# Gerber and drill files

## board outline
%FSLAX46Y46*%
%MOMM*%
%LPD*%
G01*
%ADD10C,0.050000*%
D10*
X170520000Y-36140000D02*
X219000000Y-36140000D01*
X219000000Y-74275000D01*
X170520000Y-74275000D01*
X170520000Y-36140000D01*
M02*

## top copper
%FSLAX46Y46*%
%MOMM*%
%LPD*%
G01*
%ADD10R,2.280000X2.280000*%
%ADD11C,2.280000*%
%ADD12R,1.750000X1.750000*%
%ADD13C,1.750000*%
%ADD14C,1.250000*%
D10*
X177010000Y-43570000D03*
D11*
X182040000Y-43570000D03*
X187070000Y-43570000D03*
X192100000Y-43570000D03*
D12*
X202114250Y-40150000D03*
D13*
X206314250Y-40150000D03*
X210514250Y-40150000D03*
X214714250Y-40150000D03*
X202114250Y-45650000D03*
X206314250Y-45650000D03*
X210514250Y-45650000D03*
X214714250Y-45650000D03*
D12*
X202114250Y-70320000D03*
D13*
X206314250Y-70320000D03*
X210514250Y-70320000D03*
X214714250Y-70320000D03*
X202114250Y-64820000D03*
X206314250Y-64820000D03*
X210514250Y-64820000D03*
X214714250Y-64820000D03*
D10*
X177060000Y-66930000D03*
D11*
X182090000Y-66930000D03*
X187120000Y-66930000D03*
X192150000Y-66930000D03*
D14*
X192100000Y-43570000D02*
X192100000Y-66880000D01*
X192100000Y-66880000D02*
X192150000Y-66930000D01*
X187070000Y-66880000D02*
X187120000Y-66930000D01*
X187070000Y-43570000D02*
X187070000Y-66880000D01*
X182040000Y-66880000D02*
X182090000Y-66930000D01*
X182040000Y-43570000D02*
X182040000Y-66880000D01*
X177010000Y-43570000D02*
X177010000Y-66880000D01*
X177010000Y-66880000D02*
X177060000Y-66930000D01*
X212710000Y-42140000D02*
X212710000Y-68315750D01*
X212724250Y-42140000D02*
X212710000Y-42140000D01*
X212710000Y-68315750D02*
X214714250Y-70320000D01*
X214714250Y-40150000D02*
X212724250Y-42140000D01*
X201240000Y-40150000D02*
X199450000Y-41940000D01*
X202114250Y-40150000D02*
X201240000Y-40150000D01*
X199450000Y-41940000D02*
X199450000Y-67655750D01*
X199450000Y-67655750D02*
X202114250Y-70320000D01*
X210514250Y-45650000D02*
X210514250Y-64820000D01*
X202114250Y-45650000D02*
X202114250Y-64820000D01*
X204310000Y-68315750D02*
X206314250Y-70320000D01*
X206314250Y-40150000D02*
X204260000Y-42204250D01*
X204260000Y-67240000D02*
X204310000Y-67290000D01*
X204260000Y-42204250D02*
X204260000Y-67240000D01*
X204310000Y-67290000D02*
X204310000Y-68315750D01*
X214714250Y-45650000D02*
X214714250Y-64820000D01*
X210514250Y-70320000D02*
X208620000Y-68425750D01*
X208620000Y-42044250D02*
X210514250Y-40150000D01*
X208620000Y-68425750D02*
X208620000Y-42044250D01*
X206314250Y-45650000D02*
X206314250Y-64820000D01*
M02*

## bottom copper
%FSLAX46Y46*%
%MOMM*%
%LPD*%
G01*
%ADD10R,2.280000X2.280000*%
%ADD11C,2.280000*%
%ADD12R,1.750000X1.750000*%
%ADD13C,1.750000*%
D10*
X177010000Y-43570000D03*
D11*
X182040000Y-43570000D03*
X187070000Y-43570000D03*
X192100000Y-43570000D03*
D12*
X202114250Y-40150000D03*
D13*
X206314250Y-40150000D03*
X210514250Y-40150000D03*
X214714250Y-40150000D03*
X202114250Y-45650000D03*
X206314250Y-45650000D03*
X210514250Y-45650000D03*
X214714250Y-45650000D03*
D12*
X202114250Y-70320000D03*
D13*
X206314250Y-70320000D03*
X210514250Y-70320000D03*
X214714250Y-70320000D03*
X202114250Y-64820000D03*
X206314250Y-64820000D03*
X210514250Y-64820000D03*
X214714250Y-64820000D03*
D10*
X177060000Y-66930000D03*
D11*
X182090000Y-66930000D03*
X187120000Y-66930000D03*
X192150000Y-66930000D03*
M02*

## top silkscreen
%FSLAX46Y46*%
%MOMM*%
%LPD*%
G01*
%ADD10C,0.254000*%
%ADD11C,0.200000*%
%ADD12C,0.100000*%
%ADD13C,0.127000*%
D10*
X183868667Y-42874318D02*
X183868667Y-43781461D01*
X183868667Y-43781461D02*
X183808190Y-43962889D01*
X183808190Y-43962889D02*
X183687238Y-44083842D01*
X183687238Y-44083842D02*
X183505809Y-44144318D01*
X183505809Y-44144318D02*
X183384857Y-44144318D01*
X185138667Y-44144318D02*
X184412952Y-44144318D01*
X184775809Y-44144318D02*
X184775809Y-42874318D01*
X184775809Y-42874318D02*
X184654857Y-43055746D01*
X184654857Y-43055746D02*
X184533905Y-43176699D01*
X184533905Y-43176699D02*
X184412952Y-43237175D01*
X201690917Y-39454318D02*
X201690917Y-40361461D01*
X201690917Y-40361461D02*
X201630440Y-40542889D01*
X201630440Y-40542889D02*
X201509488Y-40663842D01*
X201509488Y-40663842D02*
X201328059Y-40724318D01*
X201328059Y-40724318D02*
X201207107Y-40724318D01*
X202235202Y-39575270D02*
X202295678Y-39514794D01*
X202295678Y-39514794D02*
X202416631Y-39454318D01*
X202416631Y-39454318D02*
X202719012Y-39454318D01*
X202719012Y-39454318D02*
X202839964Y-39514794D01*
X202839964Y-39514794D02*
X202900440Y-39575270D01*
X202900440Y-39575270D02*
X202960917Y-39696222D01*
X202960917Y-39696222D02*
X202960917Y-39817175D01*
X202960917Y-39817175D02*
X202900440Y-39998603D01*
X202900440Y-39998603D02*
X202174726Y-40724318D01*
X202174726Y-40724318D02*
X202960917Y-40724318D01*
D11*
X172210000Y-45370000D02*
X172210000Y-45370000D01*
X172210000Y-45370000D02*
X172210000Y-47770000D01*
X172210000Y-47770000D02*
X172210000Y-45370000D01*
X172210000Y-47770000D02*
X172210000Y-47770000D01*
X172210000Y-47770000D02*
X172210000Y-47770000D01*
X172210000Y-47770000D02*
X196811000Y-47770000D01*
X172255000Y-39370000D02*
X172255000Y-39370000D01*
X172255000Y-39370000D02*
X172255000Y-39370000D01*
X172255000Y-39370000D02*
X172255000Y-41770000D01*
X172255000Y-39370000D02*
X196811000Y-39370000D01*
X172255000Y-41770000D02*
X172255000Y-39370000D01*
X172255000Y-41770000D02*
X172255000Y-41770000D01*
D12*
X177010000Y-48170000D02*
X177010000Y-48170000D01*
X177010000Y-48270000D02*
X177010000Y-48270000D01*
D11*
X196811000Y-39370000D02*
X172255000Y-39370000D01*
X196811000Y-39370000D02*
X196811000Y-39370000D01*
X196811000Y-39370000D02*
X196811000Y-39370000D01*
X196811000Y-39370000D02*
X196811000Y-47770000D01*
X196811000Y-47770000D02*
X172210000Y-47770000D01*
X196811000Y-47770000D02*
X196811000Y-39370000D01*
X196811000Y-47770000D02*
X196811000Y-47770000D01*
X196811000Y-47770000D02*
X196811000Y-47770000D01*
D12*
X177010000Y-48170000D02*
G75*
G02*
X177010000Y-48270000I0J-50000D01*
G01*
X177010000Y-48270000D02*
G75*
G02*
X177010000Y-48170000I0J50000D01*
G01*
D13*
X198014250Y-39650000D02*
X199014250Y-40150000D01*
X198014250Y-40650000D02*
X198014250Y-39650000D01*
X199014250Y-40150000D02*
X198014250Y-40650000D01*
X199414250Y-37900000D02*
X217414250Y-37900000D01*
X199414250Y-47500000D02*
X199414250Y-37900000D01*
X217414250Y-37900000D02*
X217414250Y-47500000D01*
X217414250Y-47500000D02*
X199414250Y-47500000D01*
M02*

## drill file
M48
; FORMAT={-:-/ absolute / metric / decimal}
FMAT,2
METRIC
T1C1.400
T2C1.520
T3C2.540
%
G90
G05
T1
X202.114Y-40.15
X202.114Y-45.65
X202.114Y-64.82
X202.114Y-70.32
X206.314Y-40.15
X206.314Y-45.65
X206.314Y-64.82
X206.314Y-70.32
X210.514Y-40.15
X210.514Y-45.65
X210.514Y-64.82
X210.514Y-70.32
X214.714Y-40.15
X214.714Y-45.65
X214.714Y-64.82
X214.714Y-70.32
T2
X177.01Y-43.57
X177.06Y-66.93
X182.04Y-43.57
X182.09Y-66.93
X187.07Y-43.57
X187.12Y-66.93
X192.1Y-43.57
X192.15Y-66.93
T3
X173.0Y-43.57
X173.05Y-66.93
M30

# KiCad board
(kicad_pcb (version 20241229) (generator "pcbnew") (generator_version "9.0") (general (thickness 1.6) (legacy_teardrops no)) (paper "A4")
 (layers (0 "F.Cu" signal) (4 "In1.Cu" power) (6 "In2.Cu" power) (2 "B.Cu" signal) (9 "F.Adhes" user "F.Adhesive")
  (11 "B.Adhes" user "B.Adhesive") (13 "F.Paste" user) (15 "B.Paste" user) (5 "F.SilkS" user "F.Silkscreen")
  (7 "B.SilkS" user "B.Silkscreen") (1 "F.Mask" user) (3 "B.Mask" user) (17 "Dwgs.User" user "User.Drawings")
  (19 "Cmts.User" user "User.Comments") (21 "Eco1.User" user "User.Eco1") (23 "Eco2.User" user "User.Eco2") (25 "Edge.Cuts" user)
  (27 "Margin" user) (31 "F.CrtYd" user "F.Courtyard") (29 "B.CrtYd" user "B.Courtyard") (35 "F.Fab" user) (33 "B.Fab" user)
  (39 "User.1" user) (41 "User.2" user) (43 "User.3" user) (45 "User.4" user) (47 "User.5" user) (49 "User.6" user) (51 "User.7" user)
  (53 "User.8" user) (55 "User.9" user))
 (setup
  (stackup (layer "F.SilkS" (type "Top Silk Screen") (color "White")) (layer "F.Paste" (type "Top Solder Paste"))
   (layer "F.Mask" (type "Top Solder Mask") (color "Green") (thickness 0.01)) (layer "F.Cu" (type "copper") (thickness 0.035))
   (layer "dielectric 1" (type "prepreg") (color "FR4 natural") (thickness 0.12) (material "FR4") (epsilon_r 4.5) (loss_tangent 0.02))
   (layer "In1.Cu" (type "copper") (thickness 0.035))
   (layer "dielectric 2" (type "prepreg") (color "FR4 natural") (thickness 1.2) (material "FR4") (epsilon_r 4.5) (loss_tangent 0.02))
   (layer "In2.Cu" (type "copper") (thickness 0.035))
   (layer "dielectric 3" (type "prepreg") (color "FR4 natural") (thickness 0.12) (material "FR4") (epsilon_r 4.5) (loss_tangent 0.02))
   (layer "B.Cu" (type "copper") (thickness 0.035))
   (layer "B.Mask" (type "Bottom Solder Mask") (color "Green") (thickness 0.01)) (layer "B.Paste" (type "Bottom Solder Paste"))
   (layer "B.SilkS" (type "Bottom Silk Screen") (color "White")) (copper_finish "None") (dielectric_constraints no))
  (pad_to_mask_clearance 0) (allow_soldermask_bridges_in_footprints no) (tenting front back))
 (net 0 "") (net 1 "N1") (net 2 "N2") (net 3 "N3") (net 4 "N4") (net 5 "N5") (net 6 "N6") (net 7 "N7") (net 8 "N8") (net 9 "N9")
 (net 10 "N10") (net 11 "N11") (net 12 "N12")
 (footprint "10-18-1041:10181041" (layer "F.Cu") (at 177.01 43.57 180)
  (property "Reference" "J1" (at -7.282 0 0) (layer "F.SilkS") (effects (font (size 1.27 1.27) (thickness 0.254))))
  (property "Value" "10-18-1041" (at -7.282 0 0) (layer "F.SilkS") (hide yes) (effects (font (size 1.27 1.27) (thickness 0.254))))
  (fp_line (start 4.8 -1.8) (end 4.8 -1.8) (stroke (width 0.2) (type solid)) (layer "F.SilkS"))
  (fp_line (start 4.8 -1.8) (end 4.8 -4.2) (stroke (width 0.2) (type solid)) (layer "F.SilkS"))
  (fp_line (start 4.8 -4.2) (end 4.8 -1.8) (stroke (width 0.2) (type solid)) (layer "F.SilkS"))
  (fp_line (start 4.8 -4.2) (end 4.8 -4.2) (stroke (width 0.2) (type solid)) (layer "F.SilkS"))
  (fp_line (start 4.8 -4.2) (end 4.8 -4.2) (stroke (width 0.2) (type solid)) (layer "F.SilkS"))
  (fp_line (start 4.8 -4.2) (end -19.801 -4.2) (stroke (width 0.2) (type solid)) (layer "F.SilkS"))
  (fp_line (start 4.755 4.2) (end 4.755 4.2) (stroke (width 0.2) (type solid)) (layer "F.SilkS"))
  (fp_line (start 4.755 4.2) (end 4.755 4.2) (stroke (width 0.2) (type solid)) (layer "F.SilkS"))
  (fp_line (start 4.755 4.2) (end 4.755 1.8) (stroke (width 0.2) (type solid)) (layer "F.SilkS"))
  (fp_line (start 4.755 4.2) (end -19.801 4.2) (stroke (width 0.2) (type solid)) (layer "F.SilkS"))
  (fp_line (start 4.755 1.8) (end 4.755 4.2) (stroke (width 0.2) (type solid)) (layer "F.SilkS"))
  (fp_line (start 4.755 1.8) (end 4.755 1.8) (stroke (width 0.2) (type solid)) (layer "F.SilkS"))
  (fp_line (start 0 -4.6) (end 0 -4.6) (stroke (width 0.1) (type solid)) (layer "F.SilkS"))
  (fp_line (start 0 -4.7) (end 0 -4.7) (stroke (width 0.1) (type solid)) (layer "F.SilkS"))
  (fp_line (start -19.801 4.2) (end 4.755 4.2) (stroke (width 0.2) (type solid)) (layer "F.SilkS"))
  (fp_line (start -19.801 4.2) (end -19.801 4.2) (stroke (width 0.2) (type solid)) (layer "F.SilkS"))
  (fp_line (start -19.801 4.2) (end -19.801 4.2) (stroke (width 0.2) (type solid)) (layer "F.SilkS"))
  (fp_line (start -19.801 4.2) (end -19.801 -4.2) (stroke (width 0.2) (type solid)) (layer "F.SilkS"))
  (fp_line (start -19.801 -4.2) (end 4.8 -4.2) (stroke (width 0.2) (type solid)) (layer "F.SilkS"))
  (fp_line (start -19.801 -4.2) (end -19.801 4.2) (stroke (width 0.2) (type solid)) (layer "F.SilkS"))
  (fp_line (start -19.801 -4.2) (end -19.801 -4.2) (stroke (width 0.2) (type solid)) (layer "F.SilkS"))
  (fp_line (start -19.801 -4.2) (end -19.801 -4.2) (stroke (width 0.2) (type solid)) (layer "F.SilkS"))
  (fp_arc (start 0 -4.6) (mid -0.05 -4.65) (end 0 -4.7) (stroke (width 0.1) (type solid)) (layer "F.SilkS"))
  (fp_arc (start 0 -4.7) (mid 0.05 -4.65) (end 0 -4.6) (stroke (width 0.1) (type solid)) (layer "F.SilkS"))
  (pad "" np_thru_hole circle (at 4.01 0 180) (size 2.54 2.54) (drill 2.54) (layers "*.Cu" "*.Mask"))
  (pad "1" thru_hole rect (at 0 0 180) (size 2.28 2.28) (drill 1.52) (layers "*.Cu" "*.Mask") (remove_unused_layers no) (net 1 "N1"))
  (pad "2" thru_hole circle (at -5.03 0 180) (size 2.28 2.28) (drill 1.52) (layers "*.Cu" "*.Mask") (remove_unused_layers no) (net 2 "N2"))
  (pad "3" thru_hole circle (at -10.06 0 180) (size 2.28 2.28) (drill 1.52) (layers "*.Cu" "*.Mask") (remove_unused_layers no) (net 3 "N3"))
  (pad "4" thru_hole circle (at -15.09 0 180) (size 2.28 2.28) (drill 1.52) (layers "*.Cu" "*.Mask") (remove_unused_layers no) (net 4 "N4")))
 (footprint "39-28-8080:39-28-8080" (layer "F.Cu") (at 202.11425 40.15)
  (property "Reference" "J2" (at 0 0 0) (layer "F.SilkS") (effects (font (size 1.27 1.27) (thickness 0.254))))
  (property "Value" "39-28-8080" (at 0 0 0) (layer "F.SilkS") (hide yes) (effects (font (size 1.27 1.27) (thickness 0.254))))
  (fp_line (start -4.1 -0.5) (end -3.1 0) (stroke (width 0.127) (type solid)) (layer "F.SilkS"))
  (fp_line (start -4.1 0.5) (end -4.1 -0.5) (stroke (width 0.127) (type solid)) (layer "F.SilkS"))
  (fp_line (start -3.1 0) (end -4.1 0.5) (stroke (width 0.127) (type solid)) (layer "F.SilkS"))
  (fp_line (start -2.7 -2.25) (end 15.3 -2.25) (stroke (width 0.127) (type solid)) (layer "F.SilkS"))
  (fp_line (start -2.7 7.35) (end -2.7 -2.25) (stroke (width 0.127) (type solid)) (layer "F.SilkS"))
  (fp_line (start 15.3 -2.25) (end 15.3 7.35) (stroke (width 0.127) (type solid)) (layer "F.SilkS"))
  (fp_line (start 15.3 7.35) (end -2.7 7.35) (stroke (width 0.127) (type solid)) (layer "F.SilkS"))
  (pad "1" thru_hole rect (at 0 0) (size 1.75 1.75) (drill 1.4) (layers "*.Cu" "*.Mask") (remove_unused_layers no) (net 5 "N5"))
  (pad "2" thru_hole circle (at 4.2 0) (size 1.75 1.75) (drill 1.4) (layers "*.Cu" "*.Mask") (remove_unused_layers no) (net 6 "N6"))
  (pad "3" thru_hole circle (at 8.4 0) (size 1.75 1.75) (drill 1.4) (layers "*.Cu" "*.Mask") (remove_unused_layers no) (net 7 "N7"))
  (pad "4" thru_hole circle (at 12.6 0) (size 1.75 1.75) (drill 1.4) (layers "*.Cu" "*.Mask") (remove_unused_layers no) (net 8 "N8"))
  (pad "5" thru_hole circle (at 0 5.5) (size 1.75 1.75) (drill 1.4) (layers "*.Cu" "*.Mask") (remove_unused_layers no) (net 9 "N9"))
  (pad "6" thru_hole circle (at 4.2 5.5) (size 1.75 1.75) (drill 1.4) (layers "*.Cu" "*.Mask") (remove_unused_layers no) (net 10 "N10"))
  (pad "7" thru_hole circle (at 8.4 5.5) (size 1.75 1.75) (drill 1.4) (layers "*.Cu" "*.Mask") (remove_unused_layers no) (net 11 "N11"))
  (pad "8" thru_hole circle (at 12.6 5.5) (size 1.75 1.75) (drill 1.4) (layers "*.Cu" "*.Mask") (remove_unused_layers no) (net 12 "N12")))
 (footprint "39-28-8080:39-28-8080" (layer "B.Cu") (at 202.11425 70.32)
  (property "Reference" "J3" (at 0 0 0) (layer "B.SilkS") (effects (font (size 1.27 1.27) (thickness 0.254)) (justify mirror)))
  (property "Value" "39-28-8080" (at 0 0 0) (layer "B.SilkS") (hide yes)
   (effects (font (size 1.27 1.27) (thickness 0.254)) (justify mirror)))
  (pad "1" thru_hole rect (at 0 0) (size 1.75 1.75) (drill 1.4) (layers "*.Cu" "*.Mask") (remove_unused_layers no) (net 5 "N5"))
  (pad "2" thru_hole circle (at 4.2 0) (size 1.75 1.75) (drill 1.4) (layers "*.Cu" "*.Mask") (remove_unused_layers no) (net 6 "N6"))
  (pad "3" thru_hole circle (at 8.4 0) (size 1.75 1.75) (drill 1.4) (layers "*.Cu" "*.Mask") (remove_unused_layers no) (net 7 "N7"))
  (pad "4" thru_hole circle (at 12.6 0) (size 1.75 1.75) (drill 1.4) (layers "*.Cu" "*.Mask") (remove_unused_layers no) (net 8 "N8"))
  (pad "5" thru_hole circle (at 0 -5.5) (size 1.75 1.75) (drill 1.4) (layers "*.Cu" "*.Mask") (remove_unused_layers no) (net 9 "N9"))
  (pad "6" thru_hole circle (at 4.2 -5.5) (size 1.75 1.75) (drill 1.4) (layers "*.Cu" "*.Mask") (remove_unused_layers no) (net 10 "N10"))
  (pad "7" thru_hole circle (at 8.4 -5.5) (size 1.75 1.75) (drill 1.4) (layers "*.Cu" "*.Mask") (remove_unused_layers no) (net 11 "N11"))
  (pad "8" thru_hole circle (at 12.6 -5.5) (size 1.75 1.75) (drill 1.4) (layers "*.Cu" "*.Mask") (remove_unused_layers no) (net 12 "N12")))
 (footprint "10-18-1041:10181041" (layer "B.Cu") (at 177.06 66.93 180)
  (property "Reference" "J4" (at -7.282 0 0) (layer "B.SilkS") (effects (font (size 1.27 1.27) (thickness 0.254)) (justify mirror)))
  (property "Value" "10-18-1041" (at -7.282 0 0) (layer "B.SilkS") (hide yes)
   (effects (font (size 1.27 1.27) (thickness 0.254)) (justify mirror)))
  (pad "" np_thru_hole circle (at 4.01 0 180) (size 2.54 2.54) (drill 2.54) (layers "*.Cu" "*.Mask"))
  (pad "1" thru_hole rect (at 0 0 180) (size 2.28 2.28) (drill 1.52) (layers "*.Cu" "*.Mask") (remove_unused_layers no) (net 1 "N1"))
  (pad "2" thru_hole circle (at -5.03 0 180) (size 2.28 2.28) (drill 1.52) (layers "*.Cu" "*.Mask") (remove_unused_layers no) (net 2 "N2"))
  (pad "3" thru_hole circle (at -10.06 0 180) (size 2.28 2.28) (drill 1.52) (layers "*.Cu" "*.Mask") (remove_unused_layers no) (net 3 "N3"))
  (pad "4" thru_hole circle (at -15.09 0 180) (size 2.28 2.28) (drill 1.52) (layers "*.Cu" "*.Mask") (remove_unused_layers no) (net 4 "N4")))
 (gr_rect (start 170.52 36.14) (end 219 74.275) (stroke (width 0.05) (type default)) (fill no) (layer "Edge.Cuts"))
 (segment (start 192.1 43.57) (end 192.1 66.88) (width 1.25) (layer "F.Cu") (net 4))
 (segment (start 192.1 66.88) (end 192.15 66.93) (width 1.25) (layer "F.Cu") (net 4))
 (segment (start 187.07 66.88) (end 187.12 66.93) (width 1.25) (layer "F.Cu") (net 3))
 (segment (start 187.07 43.57) (end 187.07 66.88) (width 1.25) (layer "F.Cu") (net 3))
 (segment (start 182.04 66.88) (end 182.09 66.93) (width 1.25) (layer "F.Cu") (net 2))
 (segment (start 182.04 43.57) (end 182.04 66.88) (width 1.25) (layer "F.Cu") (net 2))
 (segment (start 177.01 43.57) (end 177.01 66.88) (width 1.25) (layer "F.Cu") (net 1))
 (segment (start 177.01 66.88) (end 177.06 66.93) (width 1.25) (layer "F.Cu") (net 1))
 (segment (start 212.71 42.14) (end 212.71 68.31575) (width 1.25) (layer "F.Cu") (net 8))
 (segment (start 212.72425 42.14) (end 212.71 42.14) (width 1.25) (layer "F.Cu") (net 8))
 (segment (start 212.71 68.31575) (end 214.71425 70.32) (width 1.25) (layer "F.Cu") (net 8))
 (segment (start 214.71425 40.15) (end 212.72425 42.14) (width 1.25) (layer "F.Cu") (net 8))
 (segment (start 201.24 40.15) (end 199.45 41.94) (width 1.25) (layer "F.Cu") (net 5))
 (segment (start 202.11425 40.15) (end 201.24 40.15) (width 1.25) (layer "F.Cu") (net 5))
 (segment (start 199.45 41.94) (end 199.45 67.65575) (width 1.25) (layer "F.Cu") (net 5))
 (segment (start 199.45 67.65575) (end 202.11425 70.32) (width 1.25) (layer "F.Cu") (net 5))
 (segment (start 210.51425 45.65) (end 210.51425 64.82) (width 1.25) (layer "F.Cu") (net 11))
 (segment (start 202.11425 45.65) (end 202.11425 64.82) (width 1.25) (layer "F.Cu") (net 9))
 (segment (start 204.31 68.31575) (end 206.31425 70.32) (width 1.25) (layer "F.Cu") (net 6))
 (segment (start 206.31425 40.15) (end 204.26 42.20425) (width 1.25) (layer "F.Cu") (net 6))
 (segment (start 204.26 67.24) (end 204.31 67.29) (width 1.25) (layer "F.Cu") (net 6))
 (segment (start 204.26 42.20425) (end 204.26 67.24) (width 1.25) (layer "F.Cu") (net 6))
 (segment (start 204.31 67.29) (end 204.31 68.31575) (width 1.25) (layer "F.Cu") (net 6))
 (segment (start 214.71425 45.65) (end 214.71425 64.82) (width 1.25) (layer "F.Cu") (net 12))
 (segment (start 210.51425 70.32) (end 208.62 68.42575) (width 1.25) (layer "F.Cu") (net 7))
 (segment (start 208.62 42.04425) (end 210.51425 40.15) (width 1.25) (layer "F.Cu") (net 7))
 (segment (start 208.62 68.42575) (end 208.62 42.04425) (width 1.25) (layer "F.Cu") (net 7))
 (segment (start 206.31425 45.65) (end 206.31425 64.82) (width 1.25) (layer "F.Cu") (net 10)))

